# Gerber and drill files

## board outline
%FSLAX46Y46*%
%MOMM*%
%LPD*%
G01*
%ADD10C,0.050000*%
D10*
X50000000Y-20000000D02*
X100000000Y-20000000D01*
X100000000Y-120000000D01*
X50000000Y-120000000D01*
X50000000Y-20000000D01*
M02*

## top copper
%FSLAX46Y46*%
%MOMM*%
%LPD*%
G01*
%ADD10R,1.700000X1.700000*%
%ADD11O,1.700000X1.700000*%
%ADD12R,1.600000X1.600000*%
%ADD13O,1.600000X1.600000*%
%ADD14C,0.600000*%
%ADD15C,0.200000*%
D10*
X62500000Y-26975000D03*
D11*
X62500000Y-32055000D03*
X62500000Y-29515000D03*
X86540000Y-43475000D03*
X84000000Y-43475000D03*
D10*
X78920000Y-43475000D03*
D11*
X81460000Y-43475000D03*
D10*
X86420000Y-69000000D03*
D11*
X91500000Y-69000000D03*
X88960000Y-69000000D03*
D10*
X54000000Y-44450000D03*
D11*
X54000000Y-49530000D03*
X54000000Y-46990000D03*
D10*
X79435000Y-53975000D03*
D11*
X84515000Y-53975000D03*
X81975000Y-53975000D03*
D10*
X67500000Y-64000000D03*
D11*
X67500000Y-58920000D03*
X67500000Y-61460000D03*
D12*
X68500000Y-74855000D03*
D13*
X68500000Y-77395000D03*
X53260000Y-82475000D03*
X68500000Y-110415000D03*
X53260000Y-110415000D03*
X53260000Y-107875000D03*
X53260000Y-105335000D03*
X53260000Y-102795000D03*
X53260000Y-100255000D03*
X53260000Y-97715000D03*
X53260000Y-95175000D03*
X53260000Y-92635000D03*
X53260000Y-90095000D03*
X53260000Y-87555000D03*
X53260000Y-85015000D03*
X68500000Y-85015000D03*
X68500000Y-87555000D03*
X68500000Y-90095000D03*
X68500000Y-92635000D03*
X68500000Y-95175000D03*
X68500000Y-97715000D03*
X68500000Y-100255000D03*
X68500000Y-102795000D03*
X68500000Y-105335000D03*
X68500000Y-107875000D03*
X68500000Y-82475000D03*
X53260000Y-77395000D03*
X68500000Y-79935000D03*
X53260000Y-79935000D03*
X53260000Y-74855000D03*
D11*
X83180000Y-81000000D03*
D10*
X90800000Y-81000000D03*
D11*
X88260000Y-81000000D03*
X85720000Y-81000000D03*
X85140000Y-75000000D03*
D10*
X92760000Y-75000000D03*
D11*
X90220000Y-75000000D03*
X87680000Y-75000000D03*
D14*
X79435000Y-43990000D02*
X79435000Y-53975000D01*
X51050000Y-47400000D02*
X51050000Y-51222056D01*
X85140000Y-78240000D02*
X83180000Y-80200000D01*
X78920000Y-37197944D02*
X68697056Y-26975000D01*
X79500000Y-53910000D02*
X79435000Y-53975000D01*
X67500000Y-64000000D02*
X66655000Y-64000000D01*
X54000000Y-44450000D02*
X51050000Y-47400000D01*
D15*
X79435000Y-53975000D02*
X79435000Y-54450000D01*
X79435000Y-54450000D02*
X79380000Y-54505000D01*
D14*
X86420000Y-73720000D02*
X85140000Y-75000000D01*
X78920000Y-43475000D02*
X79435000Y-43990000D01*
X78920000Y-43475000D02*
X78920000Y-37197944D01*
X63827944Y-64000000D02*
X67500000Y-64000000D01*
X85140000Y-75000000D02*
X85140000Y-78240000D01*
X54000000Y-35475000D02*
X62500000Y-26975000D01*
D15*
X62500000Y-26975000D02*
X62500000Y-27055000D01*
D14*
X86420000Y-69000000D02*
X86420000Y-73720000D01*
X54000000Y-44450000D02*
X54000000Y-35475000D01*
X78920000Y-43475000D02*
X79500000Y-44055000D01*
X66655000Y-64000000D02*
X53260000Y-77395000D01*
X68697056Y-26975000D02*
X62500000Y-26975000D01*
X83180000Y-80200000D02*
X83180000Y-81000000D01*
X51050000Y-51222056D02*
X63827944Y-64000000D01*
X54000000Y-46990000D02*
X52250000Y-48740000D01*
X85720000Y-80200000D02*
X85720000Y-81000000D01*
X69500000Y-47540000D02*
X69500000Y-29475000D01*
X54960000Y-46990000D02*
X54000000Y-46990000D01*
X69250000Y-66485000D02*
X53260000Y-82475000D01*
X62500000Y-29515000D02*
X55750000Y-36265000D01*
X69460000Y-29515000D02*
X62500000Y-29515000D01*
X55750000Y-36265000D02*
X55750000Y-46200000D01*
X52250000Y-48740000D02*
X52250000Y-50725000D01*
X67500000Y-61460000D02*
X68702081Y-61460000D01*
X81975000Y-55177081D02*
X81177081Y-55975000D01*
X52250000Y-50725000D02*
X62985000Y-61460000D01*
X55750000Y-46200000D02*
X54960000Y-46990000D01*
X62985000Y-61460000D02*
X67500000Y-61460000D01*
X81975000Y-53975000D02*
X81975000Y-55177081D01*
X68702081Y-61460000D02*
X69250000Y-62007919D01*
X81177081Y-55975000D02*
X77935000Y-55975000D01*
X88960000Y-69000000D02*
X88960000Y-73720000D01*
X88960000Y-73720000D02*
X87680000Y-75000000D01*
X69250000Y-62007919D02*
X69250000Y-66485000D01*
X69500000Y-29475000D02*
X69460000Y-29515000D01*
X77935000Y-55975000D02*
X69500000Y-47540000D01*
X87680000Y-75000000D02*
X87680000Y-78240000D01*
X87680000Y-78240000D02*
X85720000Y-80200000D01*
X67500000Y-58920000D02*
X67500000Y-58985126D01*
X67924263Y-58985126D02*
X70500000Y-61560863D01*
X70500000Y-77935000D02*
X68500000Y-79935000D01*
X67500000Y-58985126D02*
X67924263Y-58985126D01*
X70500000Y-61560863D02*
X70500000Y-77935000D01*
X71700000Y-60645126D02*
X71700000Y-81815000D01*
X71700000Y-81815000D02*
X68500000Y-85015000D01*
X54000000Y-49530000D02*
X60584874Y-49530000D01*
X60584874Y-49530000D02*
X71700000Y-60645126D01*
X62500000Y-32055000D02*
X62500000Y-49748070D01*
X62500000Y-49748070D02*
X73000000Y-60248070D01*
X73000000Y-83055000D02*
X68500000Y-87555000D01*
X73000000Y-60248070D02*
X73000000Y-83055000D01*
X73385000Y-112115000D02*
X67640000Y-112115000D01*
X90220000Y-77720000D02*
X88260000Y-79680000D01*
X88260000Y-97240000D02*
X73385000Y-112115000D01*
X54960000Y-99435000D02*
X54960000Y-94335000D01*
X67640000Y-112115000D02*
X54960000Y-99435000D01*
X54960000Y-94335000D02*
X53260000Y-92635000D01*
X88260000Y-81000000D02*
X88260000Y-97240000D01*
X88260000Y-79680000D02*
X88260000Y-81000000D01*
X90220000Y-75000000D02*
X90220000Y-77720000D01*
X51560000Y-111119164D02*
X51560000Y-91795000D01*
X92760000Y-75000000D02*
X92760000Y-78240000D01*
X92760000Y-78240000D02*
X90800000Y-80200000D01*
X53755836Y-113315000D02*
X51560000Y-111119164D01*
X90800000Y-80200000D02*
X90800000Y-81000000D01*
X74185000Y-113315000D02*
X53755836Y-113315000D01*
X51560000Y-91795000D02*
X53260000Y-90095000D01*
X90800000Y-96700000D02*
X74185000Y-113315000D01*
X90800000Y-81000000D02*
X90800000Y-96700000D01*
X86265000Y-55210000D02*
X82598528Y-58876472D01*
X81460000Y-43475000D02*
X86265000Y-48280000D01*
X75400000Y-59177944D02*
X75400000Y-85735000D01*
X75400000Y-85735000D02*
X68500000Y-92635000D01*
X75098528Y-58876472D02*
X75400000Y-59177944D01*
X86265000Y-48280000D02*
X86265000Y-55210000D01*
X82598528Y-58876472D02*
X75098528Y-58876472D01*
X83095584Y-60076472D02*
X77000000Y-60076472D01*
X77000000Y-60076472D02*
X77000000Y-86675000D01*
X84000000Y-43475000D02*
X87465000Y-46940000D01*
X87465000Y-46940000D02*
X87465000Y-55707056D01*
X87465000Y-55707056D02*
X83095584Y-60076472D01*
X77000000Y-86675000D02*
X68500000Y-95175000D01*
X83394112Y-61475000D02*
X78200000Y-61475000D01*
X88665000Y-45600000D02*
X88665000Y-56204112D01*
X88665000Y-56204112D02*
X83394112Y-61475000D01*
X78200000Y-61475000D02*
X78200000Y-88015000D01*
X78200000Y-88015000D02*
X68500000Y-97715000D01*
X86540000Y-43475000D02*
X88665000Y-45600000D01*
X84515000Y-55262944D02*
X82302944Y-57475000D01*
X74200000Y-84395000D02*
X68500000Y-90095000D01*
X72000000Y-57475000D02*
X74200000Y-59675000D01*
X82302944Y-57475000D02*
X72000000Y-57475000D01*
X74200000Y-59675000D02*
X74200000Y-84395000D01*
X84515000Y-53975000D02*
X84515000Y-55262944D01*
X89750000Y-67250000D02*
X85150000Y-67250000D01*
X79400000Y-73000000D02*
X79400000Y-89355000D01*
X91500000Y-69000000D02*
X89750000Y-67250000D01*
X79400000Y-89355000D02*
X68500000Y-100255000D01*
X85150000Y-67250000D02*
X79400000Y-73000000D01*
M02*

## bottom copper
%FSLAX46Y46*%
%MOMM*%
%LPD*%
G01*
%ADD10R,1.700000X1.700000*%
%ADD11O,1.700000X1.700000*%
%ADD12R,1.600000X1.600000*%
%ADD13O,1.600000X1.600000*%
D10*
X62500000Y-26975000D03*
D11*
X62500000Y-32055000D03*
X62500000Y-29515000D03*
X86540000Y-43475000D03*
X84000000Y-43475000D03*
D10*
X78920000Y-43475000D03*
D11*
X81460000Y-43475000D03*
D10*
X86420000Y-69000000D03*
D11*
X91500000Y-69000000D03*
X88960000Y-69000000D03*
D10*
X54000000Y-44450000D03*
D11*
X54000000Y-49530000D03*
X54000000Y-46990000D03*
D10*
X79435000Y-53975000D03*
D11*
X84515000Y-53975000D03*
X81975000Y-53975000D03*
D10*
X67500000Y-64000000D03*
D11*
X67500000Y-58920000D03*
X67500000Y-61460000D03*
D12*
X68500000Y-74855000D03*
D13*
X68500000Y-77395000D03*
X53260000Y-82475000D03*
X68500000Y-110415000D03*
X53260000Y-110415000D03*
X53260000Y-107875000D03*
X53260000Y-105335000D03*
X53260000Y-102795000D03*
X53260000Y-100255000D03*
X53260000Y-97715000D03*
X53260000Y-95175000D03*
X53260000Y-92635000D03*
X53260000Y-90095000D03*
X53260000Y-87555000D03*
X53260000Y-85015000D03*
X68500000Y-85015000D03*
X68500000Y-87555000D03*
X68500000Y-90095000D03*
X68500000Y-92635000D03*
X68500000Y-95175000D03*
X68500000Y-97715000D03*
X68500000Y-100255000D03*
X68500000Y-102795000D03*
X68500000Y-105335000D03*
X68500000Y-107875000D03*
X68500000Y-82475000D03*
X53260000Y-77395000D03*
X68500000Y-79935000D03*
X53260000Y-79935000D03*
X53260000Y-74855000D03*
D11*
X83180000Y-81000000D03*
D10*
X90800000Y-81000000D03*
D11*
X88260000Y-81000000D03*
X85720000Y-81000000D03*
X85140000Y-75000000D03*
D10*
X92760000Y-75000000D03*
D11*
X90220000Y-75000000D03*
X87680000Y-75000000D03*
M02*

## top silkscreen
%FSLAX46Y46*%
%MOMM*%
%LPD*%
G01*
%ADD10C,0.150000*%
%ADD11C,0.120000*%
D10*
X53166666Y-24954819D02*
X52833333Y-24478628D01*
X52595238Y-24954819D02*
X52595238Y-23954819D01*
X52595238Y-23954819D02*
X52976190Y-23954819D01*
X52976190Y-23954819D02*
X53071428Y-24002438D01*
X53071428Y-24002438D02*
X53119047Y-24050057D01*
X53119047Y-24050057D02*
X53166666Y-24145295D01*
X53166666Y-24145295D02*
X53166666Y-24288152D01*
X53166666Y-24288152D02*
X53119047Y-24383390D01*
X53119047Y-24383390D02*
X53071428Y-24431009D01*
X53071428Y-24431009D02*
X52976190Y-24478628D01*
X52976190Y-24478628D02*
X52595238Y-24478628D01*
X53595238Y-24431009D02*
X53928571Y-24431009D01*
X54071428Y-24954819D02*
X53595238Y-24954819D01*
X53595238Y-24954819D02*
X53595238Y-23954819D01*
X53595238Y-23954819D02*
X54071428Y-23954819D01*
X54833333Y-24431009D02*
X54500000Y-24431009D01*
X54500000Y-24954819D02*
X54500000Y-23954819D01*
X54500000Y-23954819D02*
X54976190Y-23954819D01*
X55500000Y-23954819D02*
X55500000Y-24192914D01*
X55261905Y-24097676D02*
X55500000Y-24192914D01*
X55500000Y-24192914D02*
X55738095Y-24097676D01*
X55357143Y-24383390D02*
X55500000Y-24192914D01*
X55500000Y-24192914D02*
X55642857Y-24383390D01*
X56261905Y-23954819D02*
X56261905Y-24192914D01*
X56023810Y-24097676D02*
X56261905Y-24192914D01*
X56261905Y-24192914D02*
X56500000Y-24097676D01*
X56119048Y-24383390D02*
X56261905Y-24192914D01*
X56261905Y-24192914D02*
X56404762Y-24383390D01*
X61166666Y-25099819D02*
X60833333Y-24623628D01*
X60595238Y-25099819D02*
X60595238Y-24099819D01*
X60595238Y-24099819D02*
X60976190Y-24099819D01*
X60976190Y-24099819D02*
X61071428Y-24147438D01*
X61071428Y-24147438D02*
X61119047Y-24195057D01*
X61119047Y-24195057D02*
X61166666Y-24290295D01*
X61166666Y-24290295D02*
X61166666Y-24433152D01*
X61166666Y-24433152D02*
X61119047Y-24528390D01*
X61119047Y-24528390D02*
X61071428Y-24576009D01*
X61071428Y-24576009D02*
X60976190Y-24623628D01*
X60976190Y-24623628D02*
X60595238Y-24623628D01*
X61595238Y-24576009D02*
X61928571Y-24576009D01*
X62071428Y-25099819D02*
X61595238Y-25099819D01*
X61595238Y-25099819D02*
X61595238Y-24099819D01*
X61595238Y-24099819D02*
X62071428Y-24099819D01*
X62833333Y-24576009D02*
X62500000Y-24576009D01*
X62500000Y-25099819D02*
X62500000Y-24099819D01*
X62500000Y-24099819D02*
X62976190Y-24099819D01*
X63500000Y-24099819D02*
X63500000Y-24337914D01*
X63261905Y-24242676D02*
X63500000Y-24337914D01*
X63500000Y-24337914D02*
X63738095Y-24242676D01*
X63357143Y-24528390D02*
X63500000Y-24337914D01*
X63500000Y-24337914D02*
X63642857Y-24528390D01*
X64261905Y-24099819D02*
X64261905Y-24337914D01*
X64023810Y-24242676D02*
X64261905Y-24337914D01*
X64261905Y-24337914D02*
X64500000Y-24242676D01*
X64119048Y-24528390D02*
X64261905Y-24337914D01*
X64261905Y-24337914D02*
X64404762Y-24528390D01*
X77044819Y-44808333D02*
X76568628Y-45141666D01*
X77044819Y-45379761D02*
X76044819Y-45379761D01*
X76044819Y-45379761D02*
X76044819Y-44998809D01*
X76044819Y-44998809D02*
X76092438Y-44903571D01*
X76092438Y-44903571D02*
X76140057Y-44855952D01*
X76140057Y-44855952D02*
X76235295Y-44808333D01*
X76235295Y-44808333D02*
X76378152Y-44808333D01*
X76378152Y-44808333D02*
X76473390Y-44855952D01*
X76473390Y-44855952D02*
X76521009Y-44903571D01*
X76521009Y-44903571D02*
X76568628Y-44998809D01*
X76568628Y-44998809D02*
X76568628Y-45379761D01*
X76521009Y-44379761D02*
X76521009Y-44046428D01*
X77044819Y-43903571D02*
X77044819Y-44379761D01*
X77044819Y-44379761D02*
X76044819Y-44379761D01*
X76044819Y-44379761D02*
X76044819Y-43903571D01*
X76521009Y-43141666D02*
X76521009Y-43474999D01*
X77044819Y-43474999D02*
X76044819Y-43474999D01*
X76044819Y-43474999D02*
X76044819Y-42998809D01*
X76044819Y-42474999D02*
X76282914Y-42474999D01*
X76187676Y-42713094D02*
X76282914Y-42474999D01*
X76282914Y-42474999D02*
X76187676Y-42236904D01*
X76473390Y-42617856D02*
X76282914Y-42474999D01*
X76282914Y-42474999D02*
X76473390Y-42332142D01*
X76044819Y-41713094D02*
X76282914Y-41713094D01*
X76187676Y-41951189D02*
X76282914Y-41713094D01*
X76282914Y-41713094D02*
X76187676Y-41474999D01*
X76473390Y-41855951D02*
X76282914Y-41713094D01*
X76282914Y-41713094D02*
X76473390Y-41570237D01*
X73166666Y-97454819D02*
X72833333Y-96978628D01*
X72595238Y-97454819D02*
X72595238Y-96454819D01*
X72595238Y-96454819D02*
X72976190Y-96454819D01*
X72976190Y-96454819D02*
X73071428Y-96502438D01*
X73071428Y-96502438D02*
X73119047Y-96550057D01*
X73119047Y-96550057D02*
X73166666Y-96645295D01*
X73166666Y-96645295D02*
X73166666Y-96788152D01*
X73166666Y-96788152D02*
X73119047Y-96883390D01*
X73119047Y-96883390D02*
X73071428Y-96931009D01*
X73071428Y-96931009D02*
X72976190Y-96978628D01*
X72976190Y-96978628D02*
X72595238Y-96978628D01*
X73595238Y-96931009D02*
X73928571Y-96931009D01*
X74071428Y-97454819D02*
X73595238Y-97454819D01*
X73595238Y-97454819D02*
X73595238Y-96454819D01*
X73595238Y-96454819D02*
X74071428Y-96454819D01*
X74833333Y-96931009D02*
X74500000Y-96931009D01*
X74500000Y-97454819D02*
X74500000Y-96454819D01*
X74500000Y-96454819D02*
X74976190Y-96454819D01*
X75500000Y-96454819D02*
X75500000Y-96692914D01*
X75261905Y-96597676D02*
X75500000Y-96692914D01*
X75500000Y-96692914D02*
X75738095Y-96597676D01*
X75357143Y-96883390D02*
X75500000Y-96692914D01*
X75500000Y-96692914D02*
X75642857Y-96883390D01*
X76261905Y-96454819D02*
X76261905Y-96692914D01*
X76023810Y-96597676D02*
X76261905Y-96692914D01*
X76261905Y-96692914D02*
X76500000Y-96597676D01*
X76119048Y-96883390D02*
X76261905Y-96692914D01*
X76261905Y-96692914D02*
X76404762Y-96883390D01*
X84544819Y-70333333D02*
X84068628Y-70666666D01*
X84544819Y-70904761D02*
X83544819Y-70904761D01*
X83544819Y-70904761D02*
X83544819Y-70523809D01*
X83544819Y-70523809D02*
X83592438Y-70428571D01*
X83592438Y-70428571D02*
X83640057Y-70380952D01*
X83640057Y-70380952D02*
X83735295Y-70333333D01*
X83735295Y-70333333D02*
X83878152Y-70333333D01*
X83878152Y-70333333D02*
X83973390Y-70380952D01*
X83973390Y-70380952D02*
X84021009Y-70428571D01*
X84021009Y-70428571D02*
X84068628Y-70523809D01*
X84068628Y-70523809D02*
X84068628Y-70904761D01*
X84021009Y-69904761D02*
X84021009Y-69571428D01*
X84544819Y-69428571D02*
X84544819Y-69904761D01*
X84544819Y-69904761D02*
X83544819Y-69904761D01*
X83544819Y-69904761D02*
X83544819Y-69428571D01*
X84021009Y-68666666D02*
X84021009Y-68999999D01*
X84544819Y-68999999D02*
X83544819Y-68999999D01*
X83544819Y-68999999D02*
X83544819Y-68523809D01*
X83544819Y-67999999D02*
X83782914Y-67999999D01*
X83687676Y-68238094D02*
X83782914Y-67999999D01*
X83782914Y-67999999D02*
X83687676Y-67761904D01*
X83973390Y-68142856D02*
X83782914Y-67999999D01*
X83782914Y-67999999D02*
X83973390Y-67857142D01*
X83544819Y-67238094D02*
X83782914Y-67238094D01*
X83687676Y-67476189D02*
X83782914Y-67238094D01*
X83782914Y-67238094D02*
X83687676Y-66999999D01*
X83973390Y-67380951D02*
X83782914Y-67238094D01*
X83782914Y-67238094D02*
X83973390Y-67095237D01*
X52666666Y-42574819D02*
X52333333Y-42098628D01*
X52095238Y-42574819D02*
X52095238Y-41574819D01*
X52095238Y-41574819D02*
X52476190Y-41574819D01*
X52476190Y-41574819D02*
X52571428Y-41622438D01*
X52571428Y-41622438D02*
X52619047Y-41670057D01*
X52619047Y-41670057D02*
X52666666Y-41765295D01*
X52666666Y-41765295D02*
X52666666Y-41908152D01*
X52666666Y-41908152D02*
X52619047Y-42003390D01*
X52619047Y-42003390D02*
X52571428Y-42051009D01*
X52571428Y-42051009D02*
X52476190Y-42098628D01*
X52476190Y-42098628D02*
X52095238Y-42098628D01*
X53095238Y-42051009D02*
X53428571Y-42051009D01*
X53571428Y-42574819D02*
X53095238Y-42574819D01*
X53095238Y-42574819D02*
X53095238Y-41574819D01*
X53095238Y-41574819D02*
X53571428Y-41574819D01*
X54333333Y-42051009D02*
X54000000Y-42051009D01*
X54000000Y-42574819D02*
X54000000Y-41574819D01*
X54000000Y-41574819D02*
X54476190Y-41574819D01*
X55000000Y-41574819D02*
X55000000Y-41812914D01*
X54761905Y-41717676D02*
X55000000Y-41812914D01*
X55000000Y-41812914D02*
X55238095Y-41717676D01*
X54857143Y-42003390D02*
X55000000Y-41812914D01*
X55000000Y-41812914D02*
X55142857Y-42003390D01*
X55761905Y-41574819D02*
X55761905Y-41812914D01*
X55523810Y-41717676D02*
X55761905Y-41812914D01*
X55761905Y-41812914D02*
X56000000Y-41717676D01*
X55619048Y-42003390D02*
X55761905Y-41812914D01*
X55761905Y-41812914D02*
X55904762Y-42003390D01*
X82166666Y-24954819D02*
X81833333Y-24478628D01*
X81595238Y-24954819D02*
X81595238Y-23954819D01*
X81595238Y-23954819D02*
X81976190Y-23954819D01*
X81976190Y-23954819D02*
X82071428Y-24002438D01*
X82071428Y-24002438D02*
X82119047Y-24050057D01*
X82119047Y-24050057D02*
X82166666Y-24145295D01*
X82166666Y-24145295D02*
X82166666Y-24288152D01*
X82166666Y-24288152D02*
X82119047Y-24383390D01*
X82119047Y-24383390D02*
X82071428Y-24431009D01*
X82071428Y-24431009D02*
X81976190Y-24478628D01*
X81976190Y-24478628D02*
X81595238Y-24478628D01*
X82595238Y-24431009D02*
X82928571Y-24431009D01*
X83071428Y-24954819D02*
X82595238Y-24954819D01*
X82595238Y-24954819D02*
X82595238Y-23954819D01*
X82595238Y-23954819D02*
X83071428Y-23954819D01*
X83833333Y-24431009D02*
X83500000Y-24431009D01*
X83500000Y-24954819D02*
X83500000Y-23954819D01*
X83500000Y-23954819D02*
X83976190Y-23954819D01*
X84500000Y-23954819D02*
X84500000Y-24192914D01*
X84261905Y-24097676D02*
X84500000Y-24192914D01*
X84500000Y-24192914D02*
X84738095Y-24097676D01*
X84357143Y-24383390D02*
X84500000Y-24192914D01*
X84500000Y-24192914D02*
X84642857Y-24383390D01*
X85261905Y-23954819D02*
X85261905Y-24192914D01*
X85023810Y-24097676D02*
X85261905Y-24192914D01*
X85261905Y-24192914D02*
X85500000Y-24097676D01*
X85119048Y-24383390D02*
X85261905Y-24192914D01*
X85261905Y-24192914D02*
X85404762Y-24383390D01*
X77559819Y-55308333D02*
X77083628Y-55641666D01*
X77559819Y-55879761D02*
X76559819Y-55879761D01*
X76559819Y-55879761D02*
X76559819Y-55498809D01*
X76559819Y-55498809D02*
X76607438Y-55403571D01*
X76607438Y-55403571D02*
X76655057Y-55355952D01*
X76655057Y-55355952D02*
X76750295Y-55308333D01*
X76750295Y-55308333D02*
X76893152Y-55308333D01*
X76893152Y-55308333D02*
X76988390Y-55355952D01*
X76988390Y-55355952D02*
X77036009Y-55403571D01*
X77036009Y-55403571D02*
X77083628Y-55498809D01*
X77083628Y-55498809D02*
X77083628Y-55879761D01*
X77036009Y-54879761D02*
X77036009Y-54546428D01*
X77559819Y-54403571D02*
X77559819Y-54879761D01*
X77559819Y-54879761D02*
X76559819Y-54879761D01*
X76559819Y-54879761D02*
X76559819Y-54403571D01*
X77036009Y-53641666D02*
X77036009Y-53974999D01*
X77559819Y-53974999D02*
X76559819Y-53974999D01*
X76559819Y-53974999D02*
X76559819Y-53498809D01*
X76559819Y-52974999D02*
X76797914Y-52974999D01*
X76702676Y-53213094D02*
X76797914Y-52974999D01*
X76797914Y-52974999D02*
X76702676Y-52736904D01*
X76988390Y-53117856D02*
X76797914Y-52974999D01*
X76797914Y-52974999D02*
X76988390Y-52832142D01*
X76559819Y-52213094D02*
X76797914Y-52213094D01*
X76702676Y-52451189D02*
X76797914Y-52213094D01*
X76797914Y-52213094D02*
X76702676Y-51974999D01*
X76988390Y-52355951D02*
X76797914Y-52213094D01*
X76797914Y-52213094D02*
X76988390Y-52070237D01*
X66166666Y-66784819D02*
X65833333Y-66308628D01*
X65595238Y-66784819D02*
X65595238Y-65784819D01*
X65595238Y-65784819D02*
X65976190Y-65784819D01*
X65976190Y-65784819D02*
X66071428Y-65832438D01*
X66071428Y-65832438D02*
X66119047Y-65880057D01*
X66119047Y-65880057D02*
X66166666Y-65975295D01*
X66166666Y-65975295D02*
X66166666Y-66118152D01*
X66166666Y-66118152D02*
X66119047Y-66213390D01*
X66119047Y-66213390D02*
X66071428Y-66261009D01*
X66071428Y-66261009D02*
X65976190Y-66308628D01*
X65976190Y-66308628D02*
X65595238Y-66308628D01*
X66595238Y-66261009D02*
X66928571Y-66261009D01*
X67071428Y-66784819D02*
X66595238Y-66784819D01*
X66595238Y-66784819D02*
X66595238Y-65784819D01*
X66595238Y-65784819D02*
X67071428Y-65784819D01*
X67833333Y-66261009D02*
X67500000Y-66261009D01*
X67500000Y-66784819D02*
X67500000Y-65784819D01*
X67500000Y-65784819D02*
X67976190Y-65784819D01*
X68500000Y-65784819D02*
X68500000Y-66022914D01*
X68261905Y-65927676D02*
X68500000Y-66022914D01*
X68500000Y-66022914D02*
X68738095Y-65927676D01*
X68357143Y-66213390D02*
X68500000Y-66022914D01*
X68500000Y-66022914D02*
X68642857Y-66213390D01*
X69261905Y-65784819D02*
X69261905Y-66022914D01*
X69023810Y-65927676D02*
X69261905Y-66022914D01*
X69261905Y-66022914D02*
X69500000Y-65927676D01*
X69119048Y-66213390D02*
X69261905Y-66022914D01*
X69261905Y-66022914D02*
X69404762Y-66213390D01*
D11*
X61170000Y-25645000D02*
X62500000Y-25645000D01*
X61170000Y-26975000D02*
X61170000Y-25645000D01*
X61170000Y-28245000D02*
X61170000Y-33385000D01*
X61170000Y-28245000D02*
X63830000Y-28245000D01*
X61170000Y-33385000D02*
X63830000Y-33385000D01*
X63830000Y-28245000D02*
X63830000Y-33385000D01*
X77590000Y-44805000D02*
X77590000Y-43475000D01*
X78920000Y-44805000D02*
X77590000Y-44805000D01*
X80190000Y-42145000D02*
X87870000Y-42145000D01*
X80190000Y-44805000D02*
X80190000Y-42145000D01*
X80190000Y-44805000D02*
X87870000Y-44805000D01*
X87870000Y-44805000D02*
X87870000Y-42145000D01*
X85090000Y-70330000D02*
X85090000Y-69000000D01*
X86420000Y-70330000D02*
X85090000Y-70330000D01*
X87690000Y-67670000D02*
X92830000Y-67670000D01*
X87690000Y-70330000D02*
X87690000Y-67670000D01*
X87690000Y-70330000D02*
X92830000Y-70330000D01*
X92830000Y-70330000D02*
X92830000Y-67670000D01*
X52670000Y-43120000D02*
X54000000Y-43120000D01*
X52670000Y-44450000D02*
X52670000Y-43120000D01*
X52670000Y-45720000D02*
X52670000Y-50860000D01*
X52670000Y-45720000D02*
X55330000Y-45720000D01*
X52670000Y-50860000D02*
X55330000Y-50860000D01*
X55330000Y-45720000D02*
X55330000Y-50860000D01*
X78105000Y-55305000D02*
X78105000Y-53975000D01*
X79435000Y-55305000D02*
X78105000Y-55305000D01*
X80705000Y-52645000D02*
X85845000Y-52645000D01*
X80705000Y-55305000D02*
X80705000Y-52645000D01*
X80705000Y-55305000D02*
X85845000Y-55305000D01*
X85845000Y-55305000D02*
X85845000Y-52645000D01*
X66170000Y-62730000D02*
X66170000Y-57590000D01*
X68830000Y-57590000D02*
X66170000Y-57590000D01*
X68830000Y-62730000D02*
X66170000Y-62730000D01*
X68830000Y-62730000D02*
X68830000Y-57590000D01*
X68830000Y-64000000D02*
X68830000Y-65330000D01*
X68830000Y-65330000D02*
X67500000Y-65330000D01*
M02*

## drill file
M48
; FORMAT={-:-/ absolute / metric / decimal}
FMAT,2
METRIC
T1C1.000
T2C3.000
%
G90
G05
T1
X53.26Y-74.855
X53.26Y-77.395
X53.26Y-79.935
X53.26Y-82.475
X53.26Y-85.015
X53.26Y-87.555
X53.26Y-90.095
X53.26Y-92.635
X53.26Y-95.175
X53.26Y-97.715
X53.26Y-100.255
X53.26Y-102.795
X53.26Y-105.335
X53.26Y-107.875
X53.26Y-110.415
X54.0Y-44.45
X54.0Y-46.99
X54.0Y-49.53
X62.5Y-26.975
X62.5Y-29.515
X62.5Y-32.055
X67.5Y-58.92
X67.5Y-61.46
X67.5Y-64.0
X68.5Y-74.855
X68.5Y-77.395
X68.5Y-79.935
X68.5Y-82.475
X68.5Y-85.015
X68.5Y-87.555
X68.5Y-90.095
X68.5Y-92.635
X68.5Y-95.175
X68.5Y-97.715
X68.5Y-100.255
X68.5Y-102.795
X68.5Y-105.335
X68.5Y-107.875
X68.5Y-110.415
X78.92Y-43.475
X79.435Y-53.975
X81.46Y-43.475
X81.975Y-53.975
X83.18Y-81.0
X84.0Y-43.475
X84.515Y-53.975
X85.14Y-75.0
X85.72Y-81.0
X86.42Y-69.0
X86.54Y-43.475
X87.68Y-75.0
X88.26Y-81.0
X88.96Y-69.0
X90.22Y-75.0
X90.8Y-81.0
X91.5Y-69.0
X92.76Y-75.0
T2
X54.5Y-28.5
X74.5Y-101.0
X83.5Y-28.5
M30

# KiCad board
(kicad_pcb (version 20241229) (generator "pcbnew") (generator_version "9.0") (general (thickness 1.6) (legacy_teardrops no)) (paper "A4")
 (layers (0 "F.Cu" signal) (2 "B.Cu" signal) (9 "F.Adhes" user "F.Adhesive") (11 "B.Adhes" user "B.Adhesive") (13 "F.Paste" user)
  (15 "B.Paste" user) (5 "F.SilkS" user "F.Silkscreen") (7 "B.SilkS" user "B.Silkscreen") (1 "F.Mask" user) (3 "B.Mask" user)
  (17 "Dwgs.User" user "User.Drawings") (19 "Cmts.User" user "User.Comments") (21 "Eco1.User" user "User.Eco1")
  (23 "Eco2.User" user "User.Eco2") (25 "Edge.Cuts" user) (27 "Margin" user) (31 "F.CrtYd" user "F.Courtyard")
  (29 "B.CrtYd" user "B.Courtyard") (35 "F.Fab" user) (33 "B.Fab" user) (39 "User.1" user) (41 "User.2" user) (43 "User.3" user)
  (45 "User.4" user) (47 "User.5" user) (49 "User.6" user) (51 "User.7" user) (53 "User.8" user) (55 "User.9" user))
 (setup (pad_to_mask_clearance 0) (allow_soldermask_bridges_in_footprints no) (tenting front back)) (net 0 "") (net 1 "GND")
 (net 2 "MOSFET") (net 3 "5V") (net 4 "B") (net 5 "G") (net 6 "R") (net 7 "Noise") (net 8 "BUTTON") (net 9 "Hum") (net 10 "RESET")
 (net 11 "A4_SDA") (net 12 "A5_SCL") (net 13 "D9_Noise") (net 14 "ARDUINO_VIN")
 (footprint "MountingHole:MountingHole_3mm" (layer "F.Cu") (at 54.5 28.5)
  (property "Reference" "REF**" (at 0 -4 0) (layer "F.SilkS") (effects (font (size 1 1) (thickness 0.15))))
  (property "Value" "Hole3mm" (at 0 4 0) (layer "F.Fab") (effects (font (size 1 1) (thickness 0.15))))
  (pad "" np_thru_hole circle (at 0 0) (size 3 3) (drill 3) (layers "*.Cu" "*.Mask")))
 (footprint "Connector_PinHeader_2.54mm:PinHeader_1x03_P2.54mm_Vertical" (layer "F.Cu") (at 62.5 26.975)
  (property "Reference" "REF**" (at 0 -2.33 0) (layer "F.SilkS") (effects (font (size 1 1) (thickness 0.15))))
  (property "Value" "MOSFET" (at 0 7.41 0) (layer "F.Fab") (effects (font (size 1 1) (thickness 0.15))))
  (fp_line (start -1.33 -1.33) (end 0 -1.33) (stroke (width 0.12) (type solid)) (layer "F.SilkS"))
  (fp_line (start -1.33 0) (end -1.33 -1.33) (stroke (width 0.12) (type solid)) (layer "F.SilkS"))
  (fp_line (start -1.33 1.27) (end -1.33 6.41) (stroke (width 0.12) (type solid)) (layer "F.SilkS"))
  (fp_line (start -1.33 1.27) (end 1.33 1.27) (stroke (width 0.12) (type solid)) (layer "F.SilkS"))
  (fp_line (start -1.33 6.41) (end 1.33 6.41) (stroke (width 0.12) (type solid)) (layer "F.SilkS"))
  (fp_line (start 1.33 1.27) (end 1.33 6.41) (stroke (width 0.12) (type solid)) (layer "F.SilkS"))
  (pad "GND" thru_hole rect (at 0 0) (size 1.7 1.7) (drill 1) (layers "*.Cu" "*.Mask") (remove_unused_layers no) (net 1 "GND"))
  (pad "S" thru_hole oval (at 0 5.08) (size 1.7 1.7) (drill 1) (layers "*.Cu" "*.Mask") (remove_unused_layers no) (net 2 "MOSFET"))
  (pad "VCC" thru_hole oval (at 0 2.54) (size 1.7 1.7) (drill 1) (layers "*.Cu" "*.Mask") (remove_unused_layers no) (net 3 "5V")))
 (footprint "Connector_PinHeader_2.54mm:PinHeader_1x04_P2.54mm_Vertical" (layer "F.Cu") (at 78.92 43.475 90)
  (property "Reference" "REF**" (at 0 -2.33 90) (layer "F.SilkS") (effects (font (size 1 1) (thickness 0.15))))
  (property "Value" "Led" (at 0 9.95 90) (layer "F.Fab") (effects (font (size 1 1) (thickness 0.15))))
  (fp_line (start -1.33 -1.33) (end 0 -1.33) (stroke (width 0.12) (type solid)) (layer "F.SilkS"))
  (fp_line (start -1.33 0) (end -1.33 -1.33) (stroke (width 0.12) (type solid)) (layer "F.SilkS"))
  (fp_line (start 1.33 1.27) (end 1.33 8.95) (stroke (width 0.12) (type solid)) (layer "F.SilkS"))
  (fp_line (start -1.33 1.27) (end 1.33 1.27) (stroke (width 0.12) (type solid)) (layer "F.SilkS"))
  (fp_line (start -1.33 1.27) (end -1.33 8.95) (stroke (width 0.12) (type solid)) (layer "F.SilkS"))
  (fp_line (start -1.33 8.95) (end 1.33 8.95) (stroke (width 0.12) (type solid)) (layer "F.SilkS"))
  (pad "B" thru_hole oval (at 0 7.62 90) (size 1.7 1.7) (drill 1) (layers "*.Cu" "*.Mask") (remove_unused_layers no) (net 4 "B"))
  (pad "G" thru_hole oval (at 0 5.08 90) (size 1.7 1.7) (drill 1) (layers "*.Cu" "*.Mask") (remove_unused_layers no) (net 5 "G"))
  (pad "GND" thru_hole rect (at 0 0 90) (size 1.7 1.7) (drill 1) (layers "*.Cu" "*.Mask") (remove_unused_layers no) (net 1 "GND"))
  (pad "R" thru_hole oval (at 0 2.54 90) (size 1.7 1.7) (drill 1) (layers "*.Cu" "*.Mask") (remove_unused_layers no) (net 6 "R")))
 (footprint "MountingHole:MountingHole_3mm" (layer "F.Cu") (at 74.5 101)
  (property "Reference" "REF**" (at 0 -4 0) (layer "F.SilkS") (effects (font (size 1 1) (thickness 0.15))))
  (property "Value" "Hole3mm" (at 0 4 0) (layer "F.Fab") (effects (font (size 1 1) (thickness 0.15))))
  (pad "" np_thru_hole circle (at 0 0) (size 3 3) (drill 3) (layers "*.Cu" "*.Mask")))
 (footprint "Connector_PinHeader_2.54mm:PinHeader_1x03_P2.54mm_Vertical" (layer "F.Cu") (at 86.42 69 90)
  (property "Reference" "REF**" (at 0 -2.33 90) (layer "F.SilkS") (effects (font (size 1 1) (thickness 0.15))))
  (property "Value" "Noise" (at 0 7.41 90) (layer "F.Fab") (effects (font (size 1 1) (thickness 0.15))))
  (fp_line (start -1.33 -1.33) (end 0 -1.33) (stroke (width 0.12) (type solid)) (layer "F.SilkS"))
  (fp_line (start -1.33 0) (end -1.33 -1.33) (stroke (width 0.12) (type solid)) (layer "F.SilkS"))
  (fp_line (start 1.33 1.27) (end 1.33 6.41) (stroke (width 0.12) (type solid)) (layer "F.SilkS"))
  (fp_line (start -1.33 1.27) (end 1.33 1.27) (stroke (width 0.12) (type solid)) (layer "F.SilkS"))
  (fp_line (start -1.33 1.27) (end -1.33 6.41) (stroke (width 0.12) (type solid)) (layer "F.SilkS"))
  (fp_line (start -1.33 6.41) (end 1.33 6.41) (stroke (width 0.12) (type solid)) (layer "F.SilkS"))
  (pad "GND" thru_hole rect (at 0 0 90) (size 1.7 1.7) (drill 1) (layers "*.Cu" "*.Mask") (remove_unused_layers no) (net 1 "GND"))
  (pad "S" thru_hole oval (at 0 5.08 90) (size 1.7 1.7) (drill 1) (layers "*.Cu" "*.Mask") (remove_unused_layers no) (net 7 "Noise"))
  (pad "VCC" thru_hole oval (at 0 2.54 90) (size 1.7 1.7) (drill 1) (layers "*.Cu" "*.Mask") (remove_unused_layers no) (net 3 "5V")))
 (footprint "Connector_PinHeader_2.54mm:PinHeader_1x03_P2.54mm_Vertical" (layer "F.Cu") (at 54 44.45)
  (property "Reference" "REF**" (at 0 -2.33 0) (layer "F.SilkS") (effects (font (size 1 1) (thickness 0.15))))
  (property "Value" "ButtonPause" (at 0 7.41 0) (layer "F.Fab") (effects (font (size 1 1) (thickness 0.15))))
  (fp_line (start -1.33 -1.33) (end 0 -1.33) (stroke (width 0.12) (type solid)) (layer "F.SilkS"))
  (fp_line (start -1.33 0) (end -1.33 -1.33) (stroke (width 0.12) (type solid)) (layer "F.SilkS"))
  (fp_line (start -1.33 1.27) (end -1.33 6.41) (stroke (width 0.12) (type solid)) (layer "F.SilkS"))
  (fp_line (start -1.33 1.27) (end 1.33 1.27) (stroke (width 0.12) (type solid)) (layer "F.SilkS"))
  (fp_line (start -1.33 6.41) (end 1.33 6.41) (stroke (width 0.12) (type solid)) (layer "F.SilkS"))
  (fp_line (start 1.33 1.27) (end 1.33 6.41) (stroke (width 0.12) (type solid)) (layer "F.SilkS"))
  (pad "GND" thru_hole rect (at 0 0) (size 1.7 1.7) (drill 1) (layers "*.Cu" "*.Mask") (remove_unused_layers no) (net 1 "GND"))
  (pad "S" thru_hole oval (at 0 5.08) (size 1.7 1.7) (drill 1) (layers "*.Cu" "*.Mask") (remove_unused_layers no) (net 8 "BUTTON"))
  (pad "VCC" thru_hole oval (at 0 2.54) (size 1.7 1.7) (drill 1) (layers "*.Cu" "*.Mask") (remove_unused_layers no) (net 3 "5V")))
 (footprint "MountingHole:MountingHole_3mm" (layer "F.Cu") (at 83.5 28.5)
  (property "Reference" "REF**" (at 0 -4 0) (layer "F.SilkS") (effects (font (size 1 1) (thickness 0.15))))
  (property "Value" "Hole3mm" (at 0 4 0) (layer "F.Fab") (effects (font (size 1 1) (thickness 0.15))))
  (pad "" np_thru_hole circle (at 0 0) (size 3 3) (drill 3) (layers "*.Cu" "*.Mask")))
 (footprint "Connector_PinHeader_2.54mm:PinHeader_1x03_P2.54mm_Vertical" (layer "F.Cu") (at 79.435 53.975 90)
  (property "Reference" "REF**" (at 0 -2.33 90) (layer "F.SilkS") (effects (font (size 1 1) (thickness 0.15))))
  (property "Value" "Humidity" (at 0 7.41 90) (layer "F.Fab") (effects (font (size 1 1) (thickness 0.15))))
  (fp_line (start -1.33 -1.33) (end 0 -1.33) (stroke (width 0.12) (type solid)) (layer "F.SilkS"))
  (fp_line (start -1.33 0) (end -1.33 -1.33) (stroke (width 0.12) (type solid)) (layer "F.SilkS"))
  (fp_line (start 1.33 1.27) (end 1.33 6.41) (stroke (width 0.12) (type solid)) (layer "F.SilkS"))
  (fp_line (start -1.33 1.27) (end 1.33 1.27) (stroke (width 0.12) (type solid)) (layer "F.SilkS"))
  (fp_line (start -1.33 1.27) (end -1.33 6.41) (stroke (width 0.12) (type solid)) (layer "F.SilkS"))
  (fp_line (start -1.33 6.41) (end 1.33 6.41) (stroke (width 0.12) (type solid)) (layer "F.SilkS"))
  (pad "GND" thru_hole rect (at 0 0 90) (size 1.7 1.7) (drill 1) (layers "*.Cu" "*.Mask") (remove_unused_layers no) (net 1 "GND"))
  (pad "S" thru_hole oval (at 0 5.08 90) (size 1.7 1.7) (drill 1) (layers "*.Cu" "*.Mask") (remove_unused_layers no) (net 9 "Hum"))
  (pad "VCC" thru_hole oval (at 0 2.54 90) (size 1.7 1.7) (drill 1) (layers "*.Cu" "*.Mask") (remove_unused_layers no) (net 3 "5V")))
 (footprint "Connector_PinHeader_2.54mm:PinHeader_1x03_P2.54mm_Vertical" (layer "F.Cu") (at 67.5 64 180)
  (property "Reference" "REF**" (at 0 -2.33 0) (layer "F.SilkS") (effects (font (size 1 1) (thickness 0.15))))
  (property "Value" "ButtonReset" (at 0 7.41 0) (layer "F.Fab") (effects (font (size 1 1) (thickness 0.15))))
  (fp_line (start 1.33 1.27) (end 1.33 6.41) (stroke (width 0.12) (type solid)) (layer "F.SilkS"))
  (fp_line (start -1.33 6.41) (end 1.33 6.41) (stroke (width 0.12) (type solid)) (layer "F.SilkS"))
  (fp_line (start -1.33 1.27) (end 1.33 1.27) (stroke (width 0.12) (type solid)) (layer "F.SilkS"))
  (fp_line (start -1.33 1.27) (end -1.33 6.41) (stroke (width 0.12) (type solid)) (layer "F.SilkS"))
  (fp_line (start -1.33 0) (end -1.33 -1.33) (stroke (width 0.12) (type solid)) (layer "F.SilkS"))
  (fp_line (start -1.33 -1.33) (end 0 -1.33) (stroke (width 0.12) (type solid)) (layer "F.SilkS"))
  (pad "GND" thru_hole rect (at 0 0 180) (size 1.7 1.7) (drill 1) (layers "*.Cu" "*.Mask") (remove_unused_layers no) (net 1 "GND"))
  (pad "S" thru_hole oval (at 0 5.08 180) (size 1.7 1.7) (drill 1) (layers "*.Cu" "*.Mask") (remove_unused_layers no) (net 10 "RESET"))
  (pad "VCC" thru_hole oval (at 0 2.54 180) (size 1.7 1.7) (drill 1) (layers "*.Cu" "*.Mask") (remove_unused_layers no) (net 3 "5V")))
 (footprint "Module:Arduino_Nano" (layer "B.Cu") (at 68.5 74.855 180)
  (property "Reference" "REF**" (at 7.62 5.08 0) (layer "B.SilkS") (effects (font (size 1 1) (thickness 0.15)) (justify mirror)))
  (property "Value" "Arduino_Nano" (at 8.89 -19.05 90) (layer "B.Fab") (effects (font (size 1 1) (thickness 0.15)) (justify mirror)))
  (pad "1" thru_hole rect (at 0 0 180) (size 1.6 1.6) (drill 1) (layers "*.Cu" "*.Mask") (remove_unused_layers no))
  (pad "2" thru_hole oval (at 0 -2.54 180) (size 1.6 1.6) (drill 1) (layers "*.Cu" "*.Mask") (remove_unused_layers no))
  (pad "5V" thru_hole oval (at 15.24 -7.62 180) (size 1.6 1.6) (drill 1) (layers "*.Cu" "*.Mask") (remove_unused_layers no) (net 3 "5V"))
  (pad "15" thru_hole oval (at 0 -35.56 180) (size 1.6 1.6) (drill 1) (layers "*.Cu" "*.Mask") (remove_unused_layers no))
  (pad "16" thru_hole oval (at 15.24 -35.56 180) (size 1.6 1.6) (drill 1) (layers "*.Cu" "*.Mask") (remove_unused_layers no))
  (pad "17" thru_hole oval (at 15.24 -33.02 180) (size 1.6 1.6) (drill 1) (layers "*.Cu" "*.Mask") (remove_unused_layers no))
  (pad "18" thru_hole oval (at 15.24 -30.48 180) (size 1.6 1.6) (drill 1) (layers "*.Cu" "*.Mask") (remove_unused_layers no))
  (pad "A0" thru_hole oval (at 15.24 -27.94 180) (size 1.6 1.6) (drill 1) (layers "*.Cu" "*.Mask") (remove_unused_layers no))
  (pad "A1" thru_hole oval (at 15.24 -25.4 180) (size 1.6 1.6) (drill 1) (layers "*.Cu" "*.Mask") (remove_unused_layers no))
  (pad "A2" thru_hole oval (at 15.24 -22.86 180) (size 1.6 1.6) (drill 1) (layers "*.Cu" "*.Mask") (remove_unused_layers no))
  (pad "A3" thru_hole oval (at 15.24 -20.32 180) (size 1.6 1.6) (drill 1) (layers "*.Cu" "*.Mask") (remove_unused_layers no))
  (pad "A4" thru_hole oval (at 15.24 -17.78 180) (size 1.6 1.6) (drill 1) (layers "*.Cu" "*.Mask") (remove_unused_layers no)
   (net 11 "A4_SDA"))
  (pad "A5" thru_hole oval (at 15.24 -15.24 180) (size 1.6 1.6) (drill 1) (layers "*.Cu" "*.Mask") (remove_unused_layers no)
   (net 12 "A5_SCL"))
  (pad "A6" thru_hole oval (at 15.24 -12.7 180) (size 1.6 1.6) (drill 1) (layers "*.Cu" "*.Mask") (remove_unused_layers no))
  (pad "A7" thru_hole oval (at 15.24 -10.16 180) (size 1.6 1.6) (drill 1) (layers "*.Cu" "*.Mask") (remove_unused_layers no))
  (pad "D2" thru_hole oval (at 0 -10.16 180) (size 1.6 1.6) (drill 1) (layers "*.Cu" "*.Mask") (remove_unused_layers no) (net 8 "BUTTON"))
  (pad "D3" thru_hole oval (at 0 -12.7 180) (size 1.6 1.6) (drill 1) (layers "*.Cu" "*.Mask") (remove_unused_layers no) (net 2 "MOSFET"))
  (pad "D4" thru_hole oval (at 0 -15.24 180) (size 1.6 1.6) (drill 1) (layers "*.Cu" "*.Mask") (remove_unused_layers no) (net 9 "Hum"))
  (pad "D5" thru_hole oval (at 0 -17.78 180) (size 1.6 1.6) (drill 1) (layers "*.Cu" "*.Mask") (remove_unused_layers no) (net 6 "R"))
  (pad "D6" thru_hole oval (at 0 -20.32 180) (size 1.6 1.6) (drill 1) (layers "*.Cu" "*.Mask") (remove_unused_layers no) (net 5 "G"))
  (pad "D7" thru_hole oval (at 0 -22.86 180) (size 1.6 1.6) (drill 1) (layers "*.Cu" "*.Mask") (remove_unused_layers no) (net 4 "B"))
  (pad "D8" thru_hole oval (at 0 -25.4 180) (size 1.6 1.6) (drill 1) (layers "*.Cu" "*.Mask") (remove_unused_layers no) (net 7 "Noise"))
  (pad "D9" thru_hole oval (at 0 -27.94 180) (size 1.6 1.6) (drill 1) (layers "*.Cu" "*.Mask") (remove_unused_layers no) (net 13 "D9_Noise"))
  (pad "D10" thru_hole oval (at 0 -30.48 180) (size 1.6 1.6) (drill 1) (layers "*.Cu" "*.Mask") (remove_unused_layers no))
  (pad "D11" thru_hole oval (at 0 -33.02 180) (size 1.6 1.6) (drill 1) (layers "*.Cu" "*.Mask") (remove_unused_layers no))
  (pad "GND" thru_hole oval (at 0 -7.62 180) (size 1.6 1.6) (drill 1) (layers "*.Cu" "*.Mask") (remove_unused_layers no) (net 1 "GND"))
  (pad "GND" thru_hole oval (at 15.24 -2.54 180) (size 1.6 1.6) (drill 1) (layers "*.Cu" "*.Mask") (remove_unused_layers no) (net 1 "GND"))
  (pad "RST" thru_hole oval (at 0 -5.08 180) (size 1.6 1.6) (drill 1) (layers "*.Cu" "*.Mask") (remove_unused_layers no) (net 10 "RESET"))
  (pad "RST" thru_hole oval (at 15.24 -5.08 180) (size 1.6 1.6) (drill 1) (layers "*.Cu" "*.Mask") (remove_unused_layers no))
  (pad "VIN" thru_hole oval (at 15.24 0 180) (size 1.6 1.6) (drill 1) (layers "*.Cu" "*.Mask") (remove_unused_layers no)
   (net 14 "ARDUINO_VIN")))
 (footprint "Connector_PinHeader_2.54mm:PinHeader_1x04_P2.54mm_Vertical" (layer "B.Cu") (at 90.8 81 90)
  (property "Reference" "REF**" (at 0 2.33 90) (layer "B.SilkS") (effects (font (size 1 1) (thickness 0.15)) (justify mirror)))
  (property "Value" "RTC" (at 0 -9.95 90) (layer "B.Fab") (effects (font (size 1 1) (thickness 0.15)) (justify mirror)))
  (pad "GND" thru_hole oval (at 0 -7.62 90) (size 1.7 1.7) (drill 1) (layers "*.Cu" "*.Mask") (remove_unused_layers no) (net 1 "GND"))
  (pad "SCL" thru_hole rect (at 0 0 90) (size 1.7 1.7) (drill 1) (layers "*.Cu" "*.Mask") (remove_unused_layers no) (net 12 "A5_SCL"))
  (pad "SDA" thru_hole oval (at 0 -2.54 90) (size 1.7 1.7) (drill 1) (layers "*.Cu" "*.Mask") (remove_unused_layers no) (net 11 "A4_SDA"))
  (pad "VCC" thru_hole oval (at 0 -5.08 90) (size 1.7 1.7) (drill 1) (layers "*.Cu" "*.Mask") (remove_unused_layers no) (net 3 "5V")))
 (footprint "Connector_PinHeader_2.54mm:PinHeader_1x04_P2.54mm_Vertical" (layer "B.Cu") (at 92.76 75 90)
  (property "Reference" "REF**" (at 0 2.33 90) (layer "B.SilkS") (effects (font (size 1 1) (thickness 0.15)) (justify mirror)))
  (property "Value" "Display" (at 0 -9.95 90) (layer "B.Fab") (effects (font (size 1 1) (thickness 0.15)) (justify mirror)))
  (pad "GND" thru_hole oval (at 0 -7.62 90) (size 1.7 1.7) (drill 1) (layers "*.Cu" "*.Mask") (remove_unused_layers no) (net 1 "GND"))
  (pad "SCL" thru_hole rect (at 0 0 90) (size 1.7 1.7) (drill 1) (layers "*.Cu" "*.Mask") (remove_unused_layers no) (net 12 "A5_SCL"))
  (pad "SDA" thru_hole oval (at 0 -2.54 90) (size 1.7 1.7) (drill 1) (layers "*.Cu" "*.Mask") (remove_unused_layers no) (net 11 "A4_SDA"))
  (pad "VCC" thru_hole oval (at 0 -5.08 90) (size 1.7 1.7) (drill 1) (layers "*.Cu" "*.Mask") (remove_unused_layers no) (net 3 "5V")))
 (gr_rect (start 50 20) (end 100 120) (stroke (width 0.05) (type default)) (fill no) (layer "Edge.Cuts"))
 (segment (start 79.435 43.99) (end 79.435 53.975) (width 0.6) (layer "F.Cu") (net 1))
 (segment (start 51.05 47.4) (end 51.05 51.222056) (width 0.6) (layer "F.Cu") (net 1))
 (segment (start 85.14 78.24) (end 83.18 80.2) (width 0.6) (layer "F.Cu") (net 1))
 (segment (start 78.92 37.197944) (end 68.697056 26.975) (width 0.6) (layer "F.Cu") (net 1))
 (segment (start 79.5 53.91) (end 79.435 53.975) (width 0.6) (layer "F.Cu") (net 1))
 (segment (start 67.5 64) (end 66.655 64) (width 0.6) (layer "F.Cu") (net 1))
 (segment (start 54 44.45) (end 51.05 47.4) (width 0.6) (layer "F.Cu") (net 1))
 (segment (start 79.435 53.975) (end 79.435 54.45) (width 0.2) (layer "F.Cu") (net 1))
 (segment (start 79.435 54.45) (end 79.38 54.505) (width 0.2) (layer "F.Cu") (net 1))
 (segment (start 86.42 73.72) (end 85.14 75) (width 0.6) (layer "F.Cu") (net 1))
 (segment (start 78.92 43.475) (end 79.435 43.99) (width 0.6) (layer "F.Cu") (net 1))
 (segment (start 78.92 43.475) (end 78.92 37.197944) (width 0.6) (layer "F.Cu") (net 1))
 (segment (start 63.827944 64) (end 67.5 64) (width 0.6) (layer "F.Cu") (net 1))
 (segment (start 85.14 75) (end 85.14 78.24) (width 0.6) (layer "F.Cu") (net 1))
 (segment (start 54 35.475) (end 62.5 26.975) (width 0.6) (layer "F.Cu") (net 1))
 (segment (start 62.5 26.975) (end 62.5 27.055) (width 0.2) (layer "F.Cu") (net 1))
 (segment (start 86.42 69) (end 86.42 73.72) (width 0.6) (layer "F.Cu") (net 1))
 (segment (start 54 44.45) (end 54 35.475) (width 0.6) (layer "F.Cu") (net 1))
 (segment (start 78.92 43.475) (end 79.5 44.055) (width 0.6) (layer "F.Cu") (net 1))
 (segment (start 66.655 64) (end 53.26 77.395) (width 0.6) (layer "F.Cu") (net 1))
 (segment (start 68.697056 26.975) (end 62.5 26.975) (width 0.6) (layer "F.Cu") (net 1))
 (segment (start 83.18 80.2) (end 83.18 81) (width 0.6) (layer "F.Cu") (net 1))
 (segment (start 51.05 51.222056) (end 63.827944 64) (width 0.6) (layer "F.Cu") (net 1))
 (segment (start 54 46.99) (end 52.25 48.74) (width 0.6) (layer "F.Cu") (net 3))
 (segment (start 85.72 80.2) (end 85.72 81) (width 0.6) (layer "F.Cu") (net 3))
 (segment (start 69.5 47.54) (end 69.5 29.475) (width 0.6) (layer "F.Cu") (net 3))
 (segment (start 54.96 46.99) (end 54 46.99) (width 0.6) (layer "F.Cu") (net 3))
 (segment (start 69.25 66.485) (end 53.26 82.475) (width 0.6) (layer "F.Cu") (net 3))
 (segment (start 62.5 29.515) (end 55.75 36.265) (width 0.6) (layer "F.Cu") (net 3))
 (segment (start 69.46 29.515) (end 62.5 29.515) (width 0.6) (layer "F.Cu") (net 3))
 (segment (start 55.75 36.265) (end 55.75 46.2) (width 0.6) (layer "F.Cu") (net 3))
 (segment (start 52.25 48.74) (end 52.25 50.725) (width 0.6) (layer "F.Cu") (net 3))
 (segment (start 67.5 61.46) (end 68.702081 61.46) (width 0.6) (layer "F.Cu") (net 3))
 (segment (start 81.975 55.177081) (end 81.177081 55.975) (width 0.6) (layer "F.Cu") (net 3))
 (segment (start 52.25 50.725) (end 62.985 61.46) (width 0.6) (layer "F.Cu") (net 3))
 (segment (start 55.75 46.2) (end 54.96 46.99) (width 0.6) (layer "F.Cu") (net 3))
 (segment (start 62.985 61.46) (end 67.5 61.46) (width 0.6) (layer "F.Cu") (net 3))
 (segment (start 81.975 53.975) (end 81.975 55.177081) (width 0.6) (layer "F.Cu") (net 3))
 (segment (start 68.702081 61.46) (end 69.25 62.007919) (width 0.6) (layer "F.Cu") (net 3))
 (segment (start 81.177081 55.975) (end 77.935 55.975) (width 0.6) (layer "F.Cu") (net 3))
 (segment (start 88.96 69) (end 88.96 73.72) (width 0.6) (layer "F.Cu") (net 3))
 (segment (start 88.96 73.72) (end 87.68 75) (width 0.6) (layer "F.Cu") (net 3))
 (segment (start 69.25 62.007919) (end 69.25 66.485) (width 0.6) (layer "F.Cu") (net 3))
 (segment (start 69.5 29.475) (end 69.46 29.515) (width 0.6) (layer "F.Cu") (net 3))
 (segment (start 77.935 55.975) (end 69.5 47.54) (width 0.6) (layer "F.Cu") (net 3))
 (segment (start 87.68 75) (end 87.68 78.24) (width 0.6) (layer "F.Cu") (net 3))
 (segment (start 87.68 78.24) (end 85.72 80.2) (width 0.6) (layer "F.Cu") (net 3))
 (segment (start 67.5 58.92) (end 67.5 58.985126) (width 0.6) (layer "F.Cu") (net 10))
 (segment (start 67.924263 58.985126) (end 70.5 61.560863) (width 0.6) (layer "F.Cu") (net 10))
 (segment (start 70.5 77.935) (end 68.5 79.935) (width 0.6) (layer "F.Cu") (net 10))
 (segment (start 67.5 58.985126) (end 67.924263 58.985126) (width 0.6) (layer "F.Cu") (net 10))
 (segment (start 70.5 61.560863) (end 70.5 77.935) (width 0.6) (layer "F.Cu") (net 10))
 (segment (start 71.7 60.645126) (end 71.7 81.815) (width 0.6) (layer "F.Cu") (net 8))
 (segment (start 71.7 81.815) (end 68.5 85.015) (width 0.6) (layer "F.Cu") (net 8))
 (segment (start 54 49.53) (end 60.584874 49.53) (width 0.6) (layer "F.Cu") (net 8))
 (segment (start 60.584874 49.53) (end 71.7 60.645126) (width 0.6) (layer "F.Cu") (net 8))
 (segment (start 62.5 32.055) (end 62.5 49.74807) (width 0.6) (layer "F.Cu") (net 2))
 (segment (start 62.5 49.74807) (end 73 60.24807) (width 0.6) (layer "F.Cu") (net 2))
 (segment (start 73 83.055) (end 68.5 87.555) (width 0.6) (layer "F.Cu") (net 2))
 (segment (start 73 60.24807) (end 73 83.055) (width 0.6) (layer "F.Cu") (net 2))
 (segment (start 73.385 112.115) (end 67.64 112.115) (width 0.6) (layer "F.Cu") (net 11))
 (segment (start 90.22 77.72) (end 88.26 79.68) (width 0.6) (layer "F.Cu") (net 11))
 (segment (start 88.26 97.24) (end 73.385 112.115) (width 0.6) (layer "F.Cu") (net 11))
 (segment (start 54.96 99.435) (end 54.96 94.335) (width 0.6) (layer "F.Cu") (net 11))
 (segment (start 67.64 112.115) (end 54.96 99.435) (width 0.6) (layer "F.Cu") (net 11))
 (segment (start 54.96 94.335) (end 53.26 92.635) (width 0.6) (layer "F.Cu") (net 11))
 (segment (start 88.26 81) (end 88.26 97.24) (width 0.6) (layer "F.Cu") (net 11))
 (segment (start 88.26 79.68) (end 88.26 81) (width 0.6) (layer "F.Cu") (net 11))
 (segment (start 90.22 75) (end 90.22 77.72) (width 0.6) (layer "F.Cu") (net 11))
 (segment (start 51.56 111.119164) (end 51.56 91.795) (width 0.6) (layer "F.Cu") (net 12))
 (segment (start 92.76 75) (end 92.76 78.24) (width 0.6) (layer "F.Cu") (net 12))
 (segment (start 92.76 78.24) (end 90.8 80.2) (width 0.6) (layer "F.Cu") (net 12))
 (segment (start 53.755836 113.315) (end 51.56 111.119164) (width 0.6) (layer "F.Cu") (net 12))
 (segment (start 90.8 80.2) (end 90.8 81) (width 0.6) (layer "F.Cu") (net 12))
 (segment (start 74.185 113.315) (end 53.755836 113.315) (width 0.6) (layer "F.Cu") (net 12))
 (segment (start 51.56 91.795) (end 53.26 90.095) (width 0.6) (layer "F.Cu") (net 12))
 (segment (start 90.8 96.7) (end 74.185 113.315) (width 0.6) (layer "F.Cu") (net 12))
 (segment (start 90.8 81) (end 90.8 96.7) (width 0.6) (layer "F.Cu") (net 12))
 (segment (start 86.265 55.21) (end 82.598528 58.876472) (width 0.6) (layer "F.Cu") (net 6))
 (segment (start 81.46 43.475) (end 86.265 48.28) (width 0.6) (layer "F.Cu") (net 6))
 (segment (start 75.4 59.177944) (end 75.4 85.735) (width 0.6) (layer "F.Cu") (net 6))
 (segment (start 75.4 85.735) (end 68.5 92.635) (width 0.6) (layer "F.Cu") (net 6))
 (segment (start 75.098528 58.876472) (end 75.4 59.177944) (width 0.6) (layer "F.Cu") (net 6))
 (segment (start 86.265 48.28) (end 86.265 55.21) (width 0.6) (layer "F.Cu") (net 6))
 (segment (start 82.598528 58.876472) (end 75.098528 58.876472) (width 0.6) (layer "F.Cu") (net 6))
 (segment (start 83.095584 60.076472) (end 77 60.076472) (width 0.6) (layer "F.Cu") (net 5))
 (segment (start 77 60.076472) (end 77 86.675) (width 0.6) (layer "F.Cu") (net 5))
 (segment (start 84 43.475) (end 87.465 46.94) (width 0.6) (layer "F.Cu") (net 5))
 (segment (start 87.465 46.94) (end 87.465 55.707056) (width 0.6) (layer "F.Cu") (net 5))
 (segment (start 87.465 55.707056) (end 83.095584 60.076472) (width 0.6) (layer "F.Cu") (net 5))
 (segment (start 77 86.675) (end 68.5 95.175) (width 0.6) (layer "F.Cu") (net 5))
 (segment (start 83.394112 61.475) (end 78.2 61.475) (width 0.6) (layer "F.Cu") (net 4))
 (segment (start 88.665 45.6) (end 88.665 56.204112) (width 0.6) (layer "F.Cu") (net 4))
 (segment (start 88.665 56.204112) (end 83.394112 61.475) (width 0.6) (layer "F.Cu") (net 4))
 (segment (start 78.2 61.475) (end 78.2 88.015) (width 0.6) (layer "F.Cu") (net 4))
 (segment (start 78.2 88.015) (end 68.5 97.715) (width 0.6) (layer "F.Cu") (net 4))
 (segment (start 86.54 43.475) (end 88.665 45.6) (width 0.6) (layer "F.Cu") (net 4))
 (segment (start 84.515 55.262944) (end 82.302944 57.475) (width 0.6) (layer "F.Cu") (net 9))
 (segment (start 74.2 84.395) (end 68.5 90.095) (width 0.6) (layer "F.Cu") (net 9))
 (segment (start 72 57.475) (end 74.2 59.675) (width 0.6) (layer "F.Cu") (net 9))
 (segment (start 82.302944 57.475) (end 72 57.475) (width 0.6) (layer "F.Cu") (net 9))
 (segment (start 74.2 59.675) (end 74.2 84.395) (width 0.6) (layer "F.Cu") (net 9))
 (segment (start 84.515 53.975) (end 84.515 55.262944) (width 0.6) (layer "F.Cu") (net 9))
 (segment (start 89.75 67.25) (end 85.15 67.25) (width 0.6) (layer "F.Cu") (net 7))
 (segment (start 79.4 73) (end 79.4 89.355) (width 0.6) (layer "F.Cu") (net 7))
 (segment (start 91.5 69) (end 89.75 67.25) (width 0.6) (layer "F.Cu") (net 7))
 (segment (start 79.4 89.355) (end 68.5 100.255) (width 0.6) (layer "F.Cu") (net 7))
 (segment (start 85.15 67.25) (end 79.4 73) (width 0.6) (layer "F.Cu") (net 7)))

